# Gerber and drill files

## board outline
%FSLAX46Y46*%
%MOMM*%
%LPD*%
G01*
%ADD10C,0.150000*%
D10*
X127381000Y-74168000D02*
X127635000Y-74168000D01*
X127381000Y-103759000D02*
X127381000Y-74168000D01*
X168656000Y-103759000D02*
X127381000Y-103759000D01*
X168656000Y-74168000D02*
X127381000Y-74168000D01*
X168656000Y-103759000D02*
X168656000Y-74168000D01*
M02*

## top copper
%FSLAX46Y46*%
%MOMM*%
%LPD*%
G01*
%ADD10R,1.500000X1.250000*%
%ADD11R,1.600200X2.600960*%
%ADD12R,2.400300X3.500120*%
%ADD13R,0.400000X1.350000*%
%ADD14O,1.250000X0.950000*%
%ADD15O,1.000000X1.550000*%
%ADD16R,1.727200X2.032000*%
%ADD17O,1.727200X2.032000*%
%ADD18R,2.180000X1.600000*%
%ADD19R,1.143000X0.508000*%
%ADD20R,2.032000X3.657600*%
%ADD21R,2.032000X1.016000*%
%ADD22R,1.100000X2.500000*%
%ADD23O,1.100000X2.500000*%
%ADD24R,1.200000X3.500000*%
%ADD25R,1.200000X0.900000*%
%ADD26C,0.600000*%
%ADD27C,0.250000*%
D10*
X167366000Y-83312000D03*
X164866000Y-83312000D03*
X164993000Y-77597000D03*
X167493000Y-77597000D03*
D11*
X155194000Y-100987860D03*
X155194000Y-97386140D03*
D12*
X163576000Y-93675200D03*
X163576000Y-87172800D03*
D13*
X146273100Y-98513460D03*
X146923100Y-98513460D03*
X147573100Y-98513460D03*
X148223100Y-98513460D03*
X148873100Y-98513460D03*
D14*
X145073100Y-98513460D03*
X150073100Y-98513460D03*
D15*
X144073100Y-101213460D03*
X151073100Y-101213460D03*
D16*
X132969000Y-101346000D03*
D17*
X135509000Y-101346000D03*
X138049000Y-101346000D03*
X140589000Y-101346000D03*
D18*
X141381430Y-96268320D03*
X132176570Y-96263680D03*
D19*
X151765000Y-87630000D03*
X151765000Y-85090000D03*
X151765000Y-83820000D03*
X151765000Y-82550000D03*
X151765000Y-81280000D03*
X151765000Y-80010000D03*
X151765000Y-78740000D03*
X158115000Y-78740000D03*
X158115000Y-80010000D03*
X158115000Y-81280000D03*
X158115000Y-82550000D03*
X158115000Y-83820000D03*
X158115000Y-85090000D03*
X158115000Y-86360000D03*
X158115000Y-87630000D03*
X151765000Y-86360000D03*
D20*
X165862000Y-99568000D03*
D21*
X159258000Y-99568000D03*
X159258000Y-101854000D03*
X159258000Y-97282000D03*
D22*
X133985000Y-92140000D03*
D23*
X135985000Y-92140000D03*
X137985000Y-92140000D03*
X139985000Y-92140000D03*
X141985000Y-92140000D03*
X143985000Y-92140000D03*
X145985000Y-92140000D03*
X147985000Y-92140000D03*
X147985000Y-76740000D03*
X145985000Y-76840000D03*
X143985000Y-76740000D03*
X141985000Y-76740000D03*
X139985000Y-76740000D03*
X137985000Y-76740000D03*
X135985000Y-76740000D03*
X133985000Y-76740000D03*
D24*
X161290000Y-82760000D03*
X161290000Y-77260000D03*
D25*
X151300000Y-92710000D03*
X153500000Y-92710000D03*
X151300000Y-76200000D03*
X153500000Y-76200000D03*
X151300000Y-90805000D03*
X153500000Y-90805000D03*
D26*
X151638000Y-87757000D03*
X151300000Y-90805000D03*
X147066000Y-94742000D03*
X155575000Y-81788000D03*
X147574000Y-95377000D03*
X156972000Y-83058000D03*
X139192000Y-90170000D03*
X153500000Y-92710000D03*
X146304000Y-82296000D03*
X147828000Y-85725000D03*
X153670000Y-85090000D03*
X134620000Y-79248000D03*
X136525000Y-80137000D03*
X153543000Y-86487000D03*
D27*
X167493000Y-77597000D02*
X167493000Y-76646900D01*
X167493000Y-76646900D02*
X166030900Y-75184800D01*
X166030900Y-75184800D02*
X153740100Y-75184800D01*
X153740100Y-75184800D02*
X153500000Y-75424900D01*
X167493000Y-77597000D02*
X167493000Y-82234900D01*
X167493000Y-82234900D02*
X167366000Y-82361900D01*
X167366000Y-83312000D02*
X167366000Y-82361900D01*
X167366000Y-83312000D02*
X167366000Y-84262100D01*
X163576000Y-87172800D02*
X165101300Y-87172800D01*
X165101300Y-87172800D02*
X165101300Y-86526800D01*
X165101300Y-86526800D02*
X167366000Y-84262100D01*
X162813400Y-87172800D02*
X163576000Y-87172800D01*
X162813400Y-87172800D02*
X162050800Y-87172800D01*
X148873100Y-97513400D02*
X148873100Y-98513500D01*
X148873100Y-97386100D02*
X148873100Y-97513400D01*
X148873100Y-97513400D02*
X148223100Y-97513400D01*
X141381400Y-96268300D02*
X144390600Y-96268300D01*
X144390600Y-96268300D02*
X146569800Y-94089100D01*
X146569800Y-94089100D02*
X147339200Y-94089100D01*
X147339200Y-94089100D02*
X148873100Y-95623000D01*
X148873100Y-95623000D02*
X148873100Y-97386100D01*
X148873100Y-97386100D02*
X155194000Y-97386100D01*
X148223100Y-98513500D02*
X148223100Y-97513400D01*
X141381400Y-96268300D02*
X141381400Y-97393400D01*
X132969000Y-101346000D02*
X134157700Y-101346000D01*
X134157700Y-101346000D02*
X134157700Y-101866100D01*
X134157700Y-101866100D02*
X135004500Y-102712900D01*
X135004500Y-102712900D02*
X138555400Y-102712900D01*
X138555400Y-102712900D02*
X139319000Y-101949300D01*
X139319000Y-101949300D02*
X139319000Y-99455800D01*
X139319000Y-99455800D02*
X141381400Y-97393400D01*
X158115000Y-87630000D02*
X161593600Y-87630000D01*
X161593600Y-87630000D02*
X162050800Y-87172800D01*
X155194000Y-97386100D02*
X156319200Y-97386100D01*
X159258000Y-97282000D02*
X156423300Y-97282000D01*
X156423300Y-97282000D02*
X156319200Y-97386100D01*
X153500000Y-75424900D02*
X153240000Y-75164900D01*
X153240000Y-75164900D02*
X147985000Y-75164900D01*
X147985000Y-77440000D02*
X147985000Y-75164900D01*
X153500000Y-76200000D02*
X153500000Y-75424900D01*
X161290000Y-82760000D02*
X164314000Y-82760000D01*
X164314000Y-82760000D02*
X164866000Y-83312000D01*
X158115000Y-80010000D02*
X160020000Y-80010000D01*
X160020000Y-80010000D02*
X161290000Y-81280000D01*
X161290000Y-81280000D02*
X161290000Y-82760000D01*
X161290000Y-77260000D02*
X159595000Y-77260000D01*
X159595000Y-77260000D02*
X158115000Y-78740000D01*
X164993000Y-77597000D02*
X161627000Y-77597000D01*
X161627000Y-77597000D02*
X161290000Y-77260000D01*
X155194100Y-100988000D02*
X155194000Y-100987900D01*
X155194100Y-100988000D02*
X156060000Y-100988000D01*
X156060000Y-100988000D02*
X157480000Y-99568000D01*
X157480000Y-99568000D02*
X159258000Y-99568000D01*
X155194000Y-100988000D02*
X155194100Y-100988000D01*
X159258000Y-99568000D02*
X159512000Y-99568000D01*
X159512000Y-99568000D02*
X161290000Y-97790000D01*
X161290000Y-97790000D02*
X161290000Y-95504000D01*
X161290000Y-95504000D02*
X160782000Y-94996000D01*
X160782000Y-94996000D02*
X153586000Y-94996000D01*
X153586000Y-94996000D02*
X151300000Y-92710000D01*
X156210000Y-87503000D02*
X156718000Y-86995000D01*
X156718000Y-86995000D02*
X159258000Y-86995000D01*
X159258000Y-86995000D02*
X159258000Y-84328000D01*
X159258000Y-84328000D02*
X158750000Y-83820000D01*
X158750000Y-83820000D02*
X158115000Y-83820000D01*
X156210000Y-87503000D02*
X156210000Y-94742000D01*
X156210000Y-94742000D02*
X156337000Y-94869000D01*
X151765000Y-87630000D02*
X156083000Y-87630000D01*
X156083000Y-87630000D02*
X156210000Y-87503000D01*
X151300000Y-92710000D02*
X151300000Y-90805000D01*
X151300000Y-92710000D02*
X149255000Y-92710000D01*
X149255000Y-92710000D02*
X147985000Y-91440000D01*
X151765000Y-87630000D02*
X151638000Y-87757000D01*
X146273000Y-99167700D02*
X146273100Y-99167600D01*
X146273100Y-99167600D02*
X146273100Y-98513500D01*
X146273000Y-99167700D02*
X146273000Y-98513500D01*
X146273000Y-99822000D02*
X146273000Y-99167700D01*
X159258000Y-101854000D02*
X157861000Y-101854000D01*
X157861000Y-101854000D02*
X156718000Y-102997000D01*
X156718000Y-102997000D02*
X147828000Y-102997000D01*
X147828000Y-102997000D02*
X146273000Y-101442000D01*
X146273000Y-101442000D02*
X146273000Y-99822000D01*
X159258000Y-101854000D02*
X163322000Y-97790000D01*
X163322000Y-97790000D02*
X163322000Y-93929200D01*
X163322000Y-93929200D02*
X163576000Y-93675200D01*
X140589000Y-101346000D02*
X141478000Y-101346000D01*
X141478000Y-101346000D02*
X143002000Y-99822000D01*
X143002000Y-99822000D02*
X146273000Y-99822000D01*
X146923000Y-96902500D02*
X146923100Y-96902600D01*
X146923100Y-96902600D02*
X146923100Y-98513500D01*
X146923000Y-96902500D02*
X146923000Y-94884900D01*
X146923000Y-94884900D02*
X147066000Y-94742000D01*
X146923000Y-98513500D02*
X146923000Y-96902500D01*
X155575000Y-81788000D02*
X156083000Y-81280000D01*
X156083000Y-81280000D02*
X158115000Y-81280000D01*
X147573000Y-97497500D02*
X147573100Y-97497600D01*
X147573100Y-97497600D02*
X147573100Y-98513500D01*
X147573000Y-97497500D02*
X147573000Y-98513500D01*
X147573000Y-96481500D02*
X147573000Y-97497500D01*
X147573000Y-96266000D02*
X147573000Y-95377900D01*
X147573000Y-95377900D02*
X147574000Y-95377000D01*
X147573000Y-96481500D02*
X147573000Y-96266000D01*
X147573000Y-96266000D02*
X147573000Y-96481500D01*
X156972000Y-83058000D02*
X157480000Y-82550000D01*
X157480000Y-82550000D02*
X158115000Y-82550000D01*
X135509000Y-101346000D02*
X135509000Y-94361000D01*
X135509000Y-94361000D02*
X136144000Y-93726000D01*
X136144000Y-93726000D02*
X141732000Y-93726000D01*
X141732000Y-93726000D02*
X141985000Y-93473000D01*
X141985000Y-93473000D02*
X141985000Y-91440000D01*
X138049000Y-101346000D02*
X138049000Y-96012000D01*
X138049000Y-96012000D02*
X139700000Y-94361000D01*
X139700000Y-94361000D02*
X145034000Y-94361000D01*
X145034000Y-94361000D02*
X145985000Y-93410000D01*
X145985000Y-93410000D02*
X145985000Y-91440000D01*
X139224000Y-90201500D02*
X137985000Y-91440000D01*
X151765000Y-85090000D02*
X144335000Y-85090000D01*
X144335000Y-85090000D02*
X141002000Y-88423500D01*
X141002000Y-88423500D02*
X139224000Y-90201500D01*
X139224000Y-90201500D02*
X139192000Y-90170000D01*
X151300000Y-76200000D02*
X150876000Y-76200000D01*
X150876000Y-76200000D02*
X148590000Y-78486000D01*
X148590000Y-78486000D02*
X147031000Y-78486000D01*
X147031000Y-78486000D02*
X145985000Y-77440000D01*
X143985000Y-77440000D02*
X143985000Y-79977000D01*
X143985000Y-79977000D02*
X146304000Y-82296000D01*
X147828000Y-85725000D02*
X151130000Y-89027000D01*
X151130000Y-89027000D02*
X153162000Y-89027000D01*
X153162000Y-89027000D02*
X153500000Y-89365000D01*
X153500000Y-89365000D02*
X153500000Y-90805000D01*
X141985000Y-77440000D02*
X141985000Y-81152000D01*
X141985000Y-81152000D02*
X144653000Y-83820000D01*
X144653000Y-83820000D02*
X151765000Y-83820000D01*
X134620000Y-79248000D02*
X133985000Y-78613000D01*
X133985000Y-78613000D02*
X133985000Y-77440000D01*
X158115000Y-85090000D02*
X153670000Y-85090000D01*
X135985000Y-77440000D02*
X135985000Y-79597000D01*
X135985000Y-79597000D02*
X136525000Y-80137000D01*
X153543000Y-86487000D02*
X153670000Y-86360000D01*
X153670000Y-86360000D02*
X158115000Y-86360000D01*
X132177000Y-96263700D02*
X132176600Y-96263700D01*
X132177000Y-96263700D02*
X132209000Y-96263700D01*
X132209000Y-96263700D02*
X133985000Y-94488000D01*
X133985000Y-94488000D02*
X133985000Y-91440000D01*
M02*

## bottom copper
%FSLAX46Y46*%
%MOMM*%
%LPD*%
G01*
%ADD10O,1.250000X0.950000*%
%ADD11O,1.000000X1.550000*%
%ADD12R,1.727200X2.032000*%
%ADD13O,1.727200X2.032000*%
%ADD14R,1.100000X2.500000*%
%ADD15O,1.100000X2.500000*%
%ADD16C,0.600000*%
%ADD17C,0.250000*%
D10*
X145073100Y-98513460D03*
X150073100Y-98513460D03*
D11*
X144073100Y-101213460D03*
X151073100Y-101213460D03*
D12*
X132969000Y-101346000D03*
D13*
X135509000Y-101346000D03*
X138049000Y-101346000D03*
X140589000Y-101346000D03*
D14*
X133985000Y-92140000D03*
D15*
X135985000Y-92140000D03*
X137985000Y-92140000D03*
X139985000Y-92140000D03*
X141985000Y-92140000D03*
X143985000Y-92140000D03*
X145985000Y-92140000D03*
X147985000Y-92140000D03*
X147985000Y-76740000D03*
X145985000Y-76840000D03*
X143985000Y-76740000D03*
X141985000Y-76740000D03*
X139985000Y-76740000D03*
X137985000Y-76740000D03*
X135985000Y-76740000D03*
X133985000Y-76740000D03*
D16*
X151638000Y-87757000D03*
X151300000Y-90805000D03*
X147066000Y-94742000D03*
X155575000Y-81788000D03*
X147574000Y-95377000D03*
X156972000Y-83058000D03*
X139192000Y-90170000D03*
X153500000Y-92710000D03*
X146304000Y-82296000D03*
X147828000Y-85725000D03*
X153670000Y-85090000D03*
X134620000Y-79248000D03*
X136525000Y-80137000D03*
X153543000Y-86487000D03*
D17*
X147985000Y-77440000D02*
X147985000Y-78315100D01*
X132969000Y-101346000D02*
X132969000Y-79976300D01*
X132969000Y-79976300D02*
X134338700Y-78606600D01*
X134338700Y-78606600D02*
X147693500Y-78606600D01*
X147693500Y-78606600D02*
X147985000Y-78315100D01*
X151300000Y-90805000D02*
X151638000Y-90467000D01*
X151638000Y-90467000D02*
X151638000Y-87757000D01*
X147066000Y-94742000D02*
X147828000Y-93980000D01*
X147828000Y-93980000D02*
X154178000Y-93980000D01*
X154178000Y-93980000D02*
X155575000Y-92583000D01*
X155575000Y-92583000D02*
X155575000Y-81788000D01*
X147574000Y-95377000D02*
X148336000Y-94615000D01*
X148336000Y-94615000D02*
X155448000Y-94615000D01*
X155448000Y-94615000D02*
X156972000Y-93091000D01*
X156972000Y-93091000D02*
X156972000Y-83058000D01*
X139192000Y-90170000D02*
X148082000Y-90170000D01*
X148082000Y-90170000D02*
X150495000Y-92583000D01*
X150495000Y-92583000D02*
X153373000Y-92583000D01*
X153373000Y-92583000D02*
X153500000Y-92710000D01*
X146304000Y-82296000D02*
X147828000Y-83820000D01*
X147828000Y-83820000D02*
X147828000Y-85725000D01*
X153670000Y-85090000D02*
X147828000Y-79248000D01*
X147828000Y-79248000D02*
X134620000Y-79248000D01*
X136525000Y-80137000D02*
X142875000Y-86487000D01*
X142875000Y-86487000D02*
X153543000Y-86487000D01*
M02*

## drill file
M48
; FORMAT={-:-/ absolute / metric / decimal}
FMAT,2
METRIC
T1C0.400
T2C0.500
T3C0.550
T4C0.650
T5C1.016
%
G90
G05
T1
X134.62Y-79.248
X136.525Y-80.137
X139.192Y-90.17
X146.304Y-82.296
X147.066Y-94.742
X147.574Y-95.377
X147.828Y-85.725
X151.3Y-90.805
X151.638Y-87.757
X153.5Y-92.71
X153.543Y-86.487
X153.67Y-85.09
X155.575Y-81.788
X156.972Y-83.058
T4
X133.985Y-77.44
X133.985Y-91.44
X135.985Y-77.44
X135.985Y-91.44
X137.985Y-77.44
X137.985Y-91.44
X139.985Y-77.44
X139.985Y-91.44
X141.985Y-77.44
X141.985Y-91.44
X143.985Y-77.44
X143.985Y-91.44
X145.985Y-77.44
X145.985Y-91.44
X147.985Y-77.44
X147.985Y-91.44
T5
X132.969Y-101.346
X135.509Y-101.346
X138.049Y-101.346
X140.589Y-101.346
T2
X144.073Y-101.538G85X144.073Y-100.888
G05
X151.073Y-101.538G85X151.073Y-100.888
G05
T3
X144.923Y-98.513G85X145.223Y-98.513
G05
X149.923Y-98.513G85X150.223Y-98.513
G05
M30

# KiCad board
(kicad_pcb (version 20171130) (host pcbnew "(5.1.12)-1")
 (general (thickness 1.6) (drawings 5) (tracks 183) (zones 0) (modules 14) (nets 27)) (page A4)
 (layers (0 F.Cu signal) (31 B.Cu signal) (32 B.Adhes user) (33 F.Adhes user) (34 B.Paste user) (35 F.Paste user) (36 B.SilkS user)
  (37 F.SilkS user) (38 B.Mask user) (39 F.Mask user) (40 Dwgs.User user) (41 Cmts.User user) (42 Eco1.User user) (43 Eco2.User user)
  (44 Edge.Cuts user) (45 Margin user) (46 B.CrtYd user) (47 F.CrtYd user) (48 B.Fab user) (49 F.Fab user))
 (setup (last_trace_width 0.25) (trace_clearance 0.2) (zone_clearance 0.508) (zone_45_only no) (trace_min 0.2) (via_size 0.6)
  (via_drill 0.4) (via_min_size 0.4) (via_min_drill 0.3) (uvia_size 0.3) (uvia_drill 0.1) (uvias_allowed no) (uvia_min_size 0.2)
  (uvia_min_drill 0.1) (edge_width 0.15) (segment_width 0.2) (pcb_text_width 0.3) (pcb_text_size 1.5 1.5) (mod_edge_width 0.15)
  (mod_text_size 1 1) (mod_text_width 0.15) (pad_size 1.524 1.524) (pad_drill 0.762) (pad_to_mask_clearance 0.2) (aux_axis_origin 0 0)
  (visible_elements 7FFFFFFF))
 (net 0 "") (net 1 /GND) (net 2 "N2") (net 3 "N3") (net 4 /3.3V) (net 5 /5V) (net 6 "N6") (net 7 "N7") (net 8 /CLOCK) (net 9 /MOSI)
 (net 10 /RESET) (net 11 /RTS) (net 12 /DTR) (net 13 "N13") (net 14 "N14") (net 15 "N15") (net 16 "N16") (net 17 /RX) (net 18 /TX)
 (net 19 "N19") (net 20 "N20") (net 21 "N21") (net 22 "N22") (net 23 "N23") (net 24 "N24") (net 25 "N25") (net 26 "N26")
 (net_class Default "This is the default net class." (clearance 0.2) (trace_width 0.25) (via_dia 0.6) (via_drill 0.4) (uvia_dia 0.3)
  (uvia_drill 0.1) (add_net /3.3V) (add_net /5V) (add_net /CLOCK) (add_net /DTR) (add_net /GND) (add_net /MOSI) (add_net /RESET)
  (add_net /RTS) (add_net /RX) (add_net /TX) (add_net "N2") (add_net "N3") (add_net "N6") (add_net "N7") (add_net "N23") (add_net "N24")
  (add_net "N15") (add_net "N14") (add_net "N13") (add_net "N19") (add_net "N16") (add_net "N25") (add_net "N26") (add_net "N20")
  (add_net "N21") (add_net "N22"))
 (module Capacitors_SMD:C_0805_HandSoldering (layer F.Cu) (at 166.116 83.312 180)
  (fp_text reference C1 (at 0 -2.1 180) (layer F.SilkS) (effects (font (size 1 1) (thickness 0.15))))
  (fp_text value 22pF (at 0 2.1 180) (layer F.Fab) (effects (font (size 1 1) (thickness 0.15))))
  (pad 1 smd rect (at -1.25 0 180) (size 1.5 1.25) (layers F.Cu F.Paste F.Mask) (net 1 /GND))
  (pad 2 smd rect (at 1.25 0 180) (size 1.5 1.25) (layers F.Cu F.Paste F.Mask) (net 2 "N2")))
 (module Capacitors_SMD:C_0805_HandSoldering (layer F.Cu) (at 166.243 77.597)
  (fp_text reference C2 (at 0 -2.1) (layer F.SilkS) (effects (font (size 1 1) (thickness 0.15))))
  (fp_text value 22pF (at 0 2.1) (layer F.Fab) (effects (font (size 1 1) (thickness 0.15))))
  (pad 1 smd rect (at -1.25 0) (size 1.5 1.25) (layers F.Cu F.Paste F.Mask) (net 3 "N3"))
  (pad 2 smd rect (at 1.25 0) (size 1.5 1.25) (layers F.Cu F.Paste F.Mask) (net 1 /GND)))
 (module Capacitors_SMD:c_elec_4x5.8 (layer F.Cu) (at 155.194 99.187 270)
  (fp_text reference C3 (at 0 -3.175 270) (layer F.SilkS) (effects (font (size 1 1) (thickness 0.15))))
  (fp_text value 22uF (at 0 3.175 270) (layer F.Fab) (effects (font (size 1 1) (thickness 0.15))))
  (pad 1 smd rect (at 1.80086 0 270) (size 2.60096 1.6002) (layers F.Cu F.Paste F.Mask) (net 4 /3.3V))
  (pad 2 smd rect (at -1.80086 0 270) (size 2.60096 1.6002) (layers F.Cu F.Paste F.Mask) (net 1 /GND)))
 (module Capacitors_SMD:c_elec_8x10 (layer F.Cu) (at 163.576 90.424 270)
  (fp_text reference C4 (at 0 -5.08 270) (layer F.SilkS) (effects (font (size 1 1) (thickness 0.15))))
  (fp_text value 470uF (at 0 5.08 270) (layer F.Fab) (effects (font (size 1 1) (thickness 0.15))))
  (pad 1 smd rect (at 3.2512 0 270) (size 3.50012 2.4003) (layers F.Cu F.Paste F.Mask) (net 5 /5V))
  (pad 2 smd rect (at -3.2512 0 270) (size 3.50012 2.4003) (layers F.Cu F.Paste F.Mask) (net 1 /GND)))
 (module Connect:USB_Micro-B (layer F.Cu) (at 147.574 100.076)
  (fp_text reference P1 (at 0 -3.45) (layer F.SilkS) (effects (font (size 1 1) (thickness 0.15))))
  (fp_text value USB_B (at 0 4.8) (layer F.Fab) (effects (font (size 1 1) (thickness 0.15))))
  (pad 1 smd rect (at -1.3009 -1.56254 90) (size 1.35 0.4) (layers F.Cu F.Paste F.Mask) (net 5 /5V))
  (pad 2 smd rect (at -0.6509 -1.56254 90) (size 1.35 0.4) (layers F.Cu F.Paste F.Mask) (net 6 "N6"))
  (pad 3 smd rect (at -0.0009 -1.56254 90) (size 1.35 0.4) (layers F.Cu F.Paste F.Mask) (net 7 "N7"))
  (pad 4 smd rect (at 0.6491 -1.56254 90) (size 1.35 0.4) (layers F.Cu F.Paste F.Mask) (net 1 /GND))
  (pad 5 smd rect (at 1.2991 -1.56254 90) (size 1.35 0.4) (layers F.Cu F.Paste F.Mask) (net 1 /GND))
  (pad 6 thru_hole oval (at -2.5009 -1.56254 90) (size 0.95 1.25) (drill oval 0.55 0.85) (layers *.Cu *.Mask F.SilkS))
  (pad 6 thru_hole oval (at 2.4991 -1.56254 90) (size 0.95 1.25) (drill oval 0.55 0.85) (layers *.Cu *.Mask F.SilkS))
  (pad 6 thru_hole oval (at -3.5009 1.13746 90) (size 1.55 1) (drill oval 1.15 0.5) (layers *.Cu *.Mask F.SilkS))
  (pad 6 thru_hole oval (at 3.4991 1.13746 90) (size 1.55 1) (drill oval 1.15 0.5) (layers *.Cu *.Mask F.SilkS)))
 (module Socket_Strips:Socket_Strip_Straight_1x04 (layer F.Cu) (at 132.969 101.346)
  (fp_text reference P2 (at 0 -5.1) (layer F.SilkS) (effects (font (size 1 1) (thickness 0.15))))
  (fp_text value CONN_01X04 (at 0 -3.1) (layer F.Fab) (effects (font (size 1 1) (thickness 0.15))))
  (pad 1 thru_hole rect (at 0 0) (size 1.7272 2.032) (drill 1.016) (layers *.Cu *.Mask F.SilkS) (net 1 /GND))
  (pad 2 thru_hole oval (at 2.54 0) (size 1.7272 2.032) (drill 1.016) (layers *.Cu *.Mask F.SilkS) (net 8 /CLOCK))
  (pad 3 thru_hole oval (at 5.08 0) (size 1.7272 2.032) (drill 1.016) (layers *.Cu *.Mask F.SilkS) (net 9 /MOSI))
  (pad 4 thru_hole oval (at 7.62 0) (size 1.7272 2.032) (drill 1.016) (layers *.Cu *.Mask F.SilkS) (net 5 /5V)))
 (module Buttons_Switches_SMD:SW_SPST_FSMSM (layer F.Cu) (at 136.779 96.266 180)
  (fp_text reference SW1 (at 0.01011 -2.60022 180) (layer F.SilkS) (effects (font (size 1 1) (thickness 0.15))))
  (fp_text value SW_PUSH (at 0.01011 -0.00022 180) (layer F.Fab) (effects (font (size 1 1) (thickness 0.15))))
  (pad 1 smd rect (at -4.60243 -0.00232 180) (size 2.18 1.6) (layers F.Cu F.Paste F.Mask) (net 1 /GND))
  (pad 2 smd rect (at 4.60243 0.00232 180) (size 2.18 1.6) (layers F.Cu F.Paste F.Mask) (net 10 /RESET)))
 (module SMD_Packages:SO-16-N (layer F.Cu) (at 154.94 83.185 90)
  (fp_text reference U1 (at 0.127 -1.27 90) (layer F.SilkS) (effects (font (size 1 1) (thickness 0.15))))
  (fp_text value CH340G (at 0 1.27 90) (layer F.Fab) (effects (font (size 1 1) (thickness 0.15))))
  (pad 16 smd rect (at -4.445 -3.175 90) (size 0.508 1.143) (layers F.Cu F.Paste F.Mask) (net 4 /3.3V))
  (pad 14 smd rect (at -1.905 -3.175 90) (size 0.508 1.143) (layers F.Cu F.Paste F.Mask) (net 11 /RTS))
  (pad 13 smd rect (at -0.635 -3.175 90) (size 0.508 1.143) (layers F.Cu F.Paste F.Mask) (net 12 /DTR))
  (pad 12 smd rect (at 0.635 -3.175 90) (size 0.508 1.143) (layers F.Cu F.Paste F.Mask) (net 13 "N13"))
  (pad 11 smd rect (at 1.905 -3.175 90) (size 0.508 1.143) (layers F.Cu F.Paste F.Mask) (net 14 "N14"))
  (pad 10 smd rect (at 3.175 -3.175 90) (size 0.508 1.143) (layers F.Cu F.Paste F.Mask) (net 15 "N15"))
  (pad 9 smd rect (at 4.445 -3.175 90) (size 0.508 1.143) (layers F.Cu F.Paste F.Mask) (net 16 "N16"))
  (pad 8 smd rect (at 4.445 3.175 90) (size 0.508 1.143) (layers F.Cu F.Paste F.Mask) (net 3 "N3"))
  (pad 7 smd rect (at 3.175 3.175 90) (size 0.508 1.143) (layers F.Cu F.Paste F.Mask) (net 2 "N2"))
  (pad 6 smd rect (at 1.905 3.175 90) (size 0.508 1.143) (layers F.Cu F.Paste F.Mask) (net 6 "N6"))
  (pad 5 smd rect (at 0.635 3.175 90) (size 0.508 1.143) (layers F.Cu F.Paste F.Mask) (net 7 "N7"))
  (pad 4 smd rect (at -0.635 3.175 90) (size 0.508 1.143) (layers F.Cu F.Paste F.Mask) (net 4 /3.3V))
  (pad 3 smd rect (at -1.905 3.175 90) (size 0.508 1.143) (layers F.Cu F.Paste F.Mask) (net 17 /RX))
  (pad 2 smd rect (at -3.175 3.175 90) (size 0.508 1.143) (layers F.Cu F.Paste F.Mask) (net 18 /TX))
  (pad 1 smd rect (at -4.445 3.175 90) (size 0.508 1.143) (layers F.Cu F.Paste F.Mask) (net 1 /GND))
  (pad 15 smd rect (at -3.175 -3.175 90) (size 0.508 1.143) (layers F.Cu F.Paste F.Mask) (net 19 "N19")))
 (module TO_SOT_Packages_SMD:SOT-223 (layer F.Cu) (at 162.56 99.568 270)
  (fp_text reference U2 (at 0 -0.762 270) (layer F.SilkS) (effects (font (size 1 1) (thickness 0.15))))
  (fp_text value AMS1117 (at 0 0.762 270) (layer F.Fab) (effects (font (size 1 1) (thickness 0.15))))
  (pad 4 smd rect (at 0 -3.302 270) (size 3.6576 2.032) (layers F.Cu F.Paste F.Mask))
  (pad 2 smd rect (at 0 3.302 270) (size 1.016 2.032) (layers F.Cu F.Paste F.Mask) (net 4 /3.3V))
  (pad 3 smd rect (at 2.286 3.302 270) (size 1.016 2.032) (layers F.Cu F.Paste F.Mask) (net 5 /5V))
  (pad 1 smd rect (at -2.286 3.302 270) (size 1.016 2.032) (layers F.Cu F.Paste F.Mask) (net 1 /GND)))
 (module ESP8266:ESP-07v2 (layer F.Cu) (at 133.985 91.44 90)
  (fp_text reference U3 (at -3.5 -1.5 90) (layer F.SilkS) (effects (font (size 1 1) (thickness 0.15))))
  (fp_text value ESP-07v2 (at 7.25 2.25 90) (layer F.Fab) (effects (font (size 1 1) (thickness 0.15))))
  (pad 1 thru_hole rect (at 0 0 90) (size 2.5 1.1) (drill 0.65 (offset -0.7 0)) (layers *.Cu *.Mask F.SilkS) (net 10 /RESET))
  (pad 2 thru_hole oval (at 0 2 90) (size 2.5 1.1) (drill 0.65 (offset -0.7 0)) (layers *.Cu *.Mask F.SilkS) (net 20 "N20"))
  (pad 3 thru_hole oval (at 0 4 90) (size 2.5 1.1) (drill 0.65 (offset -0.7 0)) (layers *.Cu *.Mask F.SilkS) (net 11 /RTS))
  (pad 4 thru_hole oval (at 0 6 90) (size 2.5 1.1) (drill 0.65 (offset -0.7 0)) (layers *.Cu *.Mask F.SilkS) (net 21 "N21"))
  (pad 5 thru_hole oval (at 0 8 90) (size 2.5 1.1) (drill 0.65 (offset -0.7 0)) (layers *.Cu *.Mask F.SilkS) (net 8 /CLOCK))
  (pad 6 thru_hole oval (at 0 10 90) (size 2.5 1.1) (drill 0.65 (offset -0.7 0)) (layers *.Cu *.Mask F.SilkS) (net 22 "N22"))
  (pad 7 thru_hole oval (at 0 12 90) (size 2.5 1.1) (drill 0.65 (offset -0.7 0)) (layers *.Cu *.Mask F.SilkS) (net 9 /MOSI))
  (pad 8 thru_hole oval (at 0 14 90) (size 2.5 1.1) (drill 0.65 (offset -0.7 0)) (layers *.Cu *.Mask F.SilkS) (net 4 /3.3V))
  (pad 9 thru_hole oval (at 14 14 90) (size 2.5 1.1) (drill 0.65 (offset 0.7 0)) (layers *.Cu *.Mask F.SilkS) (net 1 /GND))
  (pad 10 thru_hole oval (at 14 12 90) (size 2.5 1.1) (drill 0.65 (offset 0.6 0)) (layers *.Cu *.Mask F.SilkS) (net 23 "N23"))
  (pad 11 thru_hole oval (at 14 10 90) (size 2.5 1.1) (drill 0.65 (offset 0.7 0)) (layers *.Cu *.Mask F.SilkS) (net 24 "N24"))
  (pad 12 thru_hole oval (at 14 8 90) (size 2.5 1.1) (drill 0.65 (offset 0.7 0)) (layers *.Cu *.Mask F.SilkS) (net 12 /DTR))
  (pad 13 thru_hole oval (at 14 6 90) (size 2.5 1.1) (drill 0.65 (offset 0.7 0)) (layers *.Cu *.Mask F.SilkS) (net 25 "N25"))
  (pad 14 thru_hole oval (at 14 4 90) (size 2.5 1.1) (drill 0.65 (offset 0.7 0)) (layers *.Cu *.Mask F.SilkS) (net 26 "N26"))
  (pad 15 thru_hole oval (at 14 2 90) (size 2.5 1.1) (drill 0.65 (offset 0.7 0)) (layers *.Cu *.Mask F.SilkS) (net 18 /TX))
  (pad 16 thru_hole oval (at 14 0 90) (size 2.5 1.1) (drill 0.65 (offset 0.7 0)) (layers *.Cu *.Mask F.SilkS) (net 17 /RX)))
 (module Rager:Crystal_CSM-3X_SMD (layer F.Cu) (at 161.29 80.01 90)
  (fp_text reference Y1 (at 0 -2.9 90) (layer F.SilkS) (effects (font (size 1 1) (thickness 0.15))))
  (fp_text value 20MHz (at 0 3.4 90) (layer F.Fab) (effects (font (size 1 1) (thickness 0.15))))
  (pad 1 smd rect (at -2.75 0 90) (size 3.5 1.2) (layers F.Cu F.Paste F.Mask) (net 2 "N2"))
  (pad 2 smd rect (at 2.75 0 90) (size 3.5 1.2) (layers F.Cu F.Paste F.Mask) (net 3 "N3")))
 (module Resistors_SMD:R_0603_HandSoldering (layer F.Cu) (at 152.4 92.71)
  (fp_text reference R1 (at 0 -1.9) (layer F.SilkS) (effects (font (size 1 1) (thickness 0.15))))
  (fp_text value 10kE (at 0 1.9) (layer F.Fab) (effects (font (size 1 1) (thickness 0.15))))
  (pad 1 smd rect (at -1.1 0) (size 1.2 0.9) (layers F.Cu F.Paste F.Mask) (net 4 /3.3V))
  (pad 2 smd rect (at 1.1 0) (size 1.2 0.9) (layers F.Cu F.Paste F.Mask) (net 11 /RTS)))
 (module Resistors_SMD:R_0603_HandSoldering (layer F.Cu) (at 152.4 76.2)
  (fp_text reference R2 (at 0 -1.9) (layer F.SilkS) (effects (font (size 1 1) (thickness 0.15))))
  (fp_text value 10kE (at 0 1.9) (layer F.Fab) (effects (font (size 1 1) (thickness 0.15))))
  (pad 1 smd rect (at -1.1 0) (size 1.2 0.9) (layers F.Cu F.Paste F.Mask) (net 23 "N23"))
  (pad 2 smd rect (at 1.1 0) (size 1.2 0.9) (layers F.Cu F.Paste F.Mask) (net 1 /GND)))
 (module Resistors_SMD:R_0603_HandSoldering (layer F.Cu) (at 152.4 90.805)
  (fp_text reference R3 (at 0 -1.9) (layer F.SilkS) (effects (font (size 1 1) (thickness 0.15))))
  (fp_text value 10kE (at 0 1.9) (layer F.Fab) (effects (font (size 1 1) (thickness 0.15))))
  (pad 1 smd rect (at -1.1 0) (size 1.2 0.9) (layers F.Cu F.Paste F.Mask) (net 4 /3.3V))
  (pad 2 smd rect (at 1.1 0) (size 1.2 0.9) (layers F.Cu F.Paste F.Mask) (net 24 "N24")))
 (gr_line (start 127.381 74.168) (end 127.635 74.168) (angle 90) (layer Edge.Cuts) (width 0.15))
 (gr_line (start 127.381 103.759) (end 127.381 74.168) (angle 90) (layer Edge.Cuts) (width 0.15))
 (gr_line (start 168.656 103.759) (end 127.381 103.759) (angle 90) (layer Edge.Cuts) (width 0.15))
 (gr_line (start 168.656 74.168) (end 127.381 74.168) (angle 90) (layer Edge.Cuts) (width 0.15))
 (gr_line (start 168.656 103.759) (end 168.656 74.168) (angle 90) (layer Edge.Cuts) (width 0.15))
 (segment (start 167.493 77.597) (end 167.493 76.6469) (width 0.25) (layer F.Cu) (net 1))
 (segment (start 167.493 76.6469) (end 166.0309 75.1848) (width 0.25) (layer F.Cu) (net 1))
 (segment (start 166.0309 75.1848) (end 153.7401 75.1848) (width 0.25) (layer F.Cu) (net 1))
 (segment (start 153.7401 75.1848) (end 153.5 75.4249) (width 0.25) (layer F.Cu) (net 1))
 (segment (start 167.493 77.597) (end 167.493 82.2349) (width 0.25) (layer F.Cu) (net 1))
 (segment (start 167.493 82.2349) (end 167.366 82.3619) (width 0.25) (layer F.Cu) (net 1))
 (segment (start 167.366 83.312) (end 167.366 82.3619) (width 0.25) (layer F.Cu) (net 1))
 (segment (start 147.985 77.44) (end 147.985 78.3151) (width 0.25) (layer B.Cu) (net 1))
 (segment (start 132.969 101.346) (end 132.969 79.9763) (width 0.25) (layer B.Cu) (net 1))
 (segment (start 132.969 79.9763) (end 134.3387 78.6066) (width 0.25) (layer B.Cu) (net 1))
 (segment (start 134.3387 78.6066) (end 147.6935 78.6066) (width 0.25) (layer B.Cu) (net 1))
 (segment (start 147.6935 78.6066) (end 147.985 78.3151) (width 0.25) (layer B.Cu) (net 1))
 (segment (start 167.366 83.312) (end 167.366 84.2621) (width 0.25) (layer F.Cu) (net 1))
 (segment (start 163.576 87.1728) (end 165.1013 87.1728) (width 0.25) (layer F.Cu) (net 1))
 (segment (start 165.1013 87.1728) (end 165.1013 86.5268) (width 0.25) (layer F.Cu) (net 1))
 (segment (start 165.1013 86.5268) (end 167.366 84.2621) (width 0.25) (layer F.Cu) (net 1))
 (segment (start 162.8134 87.1728) (end 163.576 87.1728) (width 0.25) (layer F.Cu) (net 1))
 (segment (start 162.8134 87.1728) (end 162.0508 87.1728) (width 0.25) (layer F.Cu) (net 1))
 (segment (start 148.8731 97.5134) (end 148.8731 98.5135) (width 0.25) (layer F.Cu) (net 1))
 (segment (start 148.8731 97.3861) (end 148.8731 97.5134) (width 0.25) (layer F.Cu) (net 1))
 (segment (start 148.8731 97.5134) (end 148.2231 97.5134) (width 0.25) (layer F.Cu) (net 1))
 (segment (start 141.3814 96.2683) (end 144.3906 96.2683) (width 0.25) (layer F.Cu) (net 1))
 (segment (start 144.3906 96.2683) (end 146.5698 94.0891) (width 0.25) (layer F.Cu) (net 1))
 (segment (start 146.5698 94.0891) (end 147.3392 94.0891) (width 0.25) (layer F.Cu) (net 1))
 (segment (start 147.3392 94.0891) (end 148.8731 95.623) (width 0.25) (layer F.Cu) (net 1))
 (segment (start 148.8731 95.623) (end 148.8731 97.3861) (width 0.25) (layer F.Cu) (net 1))
 (segment (start 148.8731 97.3861) (end 155.194 97.3861) (width 0.25) (layer F.Cu) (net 1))
 (segment (start 148.2231 98.5135) (end 148.2231 97.5134) (width 0.25) (layer F.Cu) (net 1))
 (segment (start 141.3814 96.2683) (end 141.3814 97.3934) (width 0.25) (layer F.Cu) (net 1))
 (segment (start 132.969 101.346) (end 134.1577 101.346) (width 0.25) (layer F.Cu) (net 1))
 (segment (start 134.1577 101.346) (end 134.1577 101.8661) (width 0.25) (layer F.Cu) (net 1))
 (segment (start 134.1577 101.8661) (end 135.0045 102.7129) (width 0.25) (layer F.Cu) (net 1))
 (segment (start 135.0045 102.7129) (end 138.5554 102.7129) (width 0.25) (layer F.Cu) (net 1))
 (segment (start 138.5554 102.7129) (end 139.319 101.9493) (width 0.25) (layer F.Cu) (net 1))
 (segment (start 139.319 101.9493) (end 139.319 99.4558) (width 0.25) (layer F.Cu) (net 1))
 (segment (start 139.319 99.4558) (end 141.3814 97.3934) (width 0.25) (layer F.Cu) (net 1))
 (segment (start 158.115 87.63) (end 161.5936 87.63) (width 0.25) (layer F.Cu) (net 1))
 (segment (start 161.5936 87.63) (end 162.0508 87.1728) (width 0.25) (layer F.Cu) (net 1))
 (segment (start 155.194 97.3861) (end 156.3192 97.3861) (width 0.25) (layer F.Cu) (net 1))
 (segment (start 159.258 97.282) (end 156.4233 97.282) (width 0.25) (layer F.Cu) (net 1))
 (segment (start 156.4233 97.282) (end 156.3192 97.3861) (width 0.25) (layer F.Cu) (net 1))
 (segment (start 153.5 75.4249) (end 153.24 75.1649) (width 0.25) (layer F.Cu) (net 1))
 (segment (start 153.24 75.1649) (end 147.985 75.1649) (width 0.25) (layer F.Cu) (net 1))
 (segment (start 147.985 77.44) (end 147.985 75.1649) (width 0.25) (layer F.Cu) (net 1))
 (segment (start 153.5 76.2) (end 153.5 75.4249) (width 0.25) (layer F.Cu) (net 1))
 (segment (start 161.29 82.76) (end 164.314 82.76) (width 0.25) (layer F.Cu) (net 2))
 (segment (start 164.314 82.76) (end 164.866 83.312) (width 0.25) (layer F.Cu) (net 2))
 (segment (start 158.115 80.01) (end 160.02 80.01) (width 0.25) (layer F.Cu) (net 2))
 (segment (start 160.02 80.01) (end 161.29 81.28) (width 0.25) (layer F.Cu) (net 2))
 (segment (start 161.29 81.28) (end 161.29 82.76) (width 0.25) (layer F.Cu) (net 2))
 (segment (start 161.29 77.26) (end 159.595 77.26) (width 0.25) (layer F.Cu) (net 3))
 (segment (start 159.595 77.26) (end 158.115 78.74) (width 0.25) (layer F.Cu) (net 3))
 (segment (start 164.993 77.597) (end 161.627 77.597) (width 0.25) (layer F.Cu) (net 3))
 (segment (start 161.627 77.597) (end 161.29 77.26) (width 0.25) (layer F.Cu) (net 3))
 (segment (start 155.1941 100.988) (end 155.194 100.9879) (width 0.25) (layer F.Cu) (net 4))
 (segment (start 155.1941 100.988) (end 156.06 100.988) (width 0.25) (layer F.Cu) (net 4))
 (segment (start 156.06 100.988) (end 157.48 99.568) (width 0.25) (layer F.Cu) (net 4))
 (segment (start 157.48 99.568) (end 159.258 99.568) (width 0.25) (layer F.Cu) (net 4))
 (segment (start 155.194 100.988) (end 155.1941 100.988) (width 0.25) (layer F.Cu) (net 4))
 (segment (start 159.258 99.568) (end 159.512 99.568) (width 0.25) (layer F.Cu) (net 4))
 (segment (start 159.512 99.568) (end 161.29 97.79) (width 0.25) (layer F.Cu) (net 4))
 (segment (start 161.29 97.79) (end 161.29 95.504) (width 0.25) (layer F.Cu) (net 4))
 (segment (start 161.29 95.504) (end 160.782 94.996) (width 0.25) (layer F.Cu) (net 4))
 (segment (start 160.782 94.996) (end 153.586 94.996) (width 0.25) (layer F.Cu) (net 4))
 (segment (start 153.586 94.996) (end 151.3 92.71) (width 0.25) (layer F.Cu) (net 4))
 (segment (start 156.21 87.503) (end 156.718 86.995) (width 0.25) (layer F.Cu) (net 4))
 (segment (start 156.718 86.995) (end 159.258 86.995) (width 0.25) (layer F.Cu) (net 4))
 (segment (start 159.258 86.995) (end 159.258 84.328) (width 0.25) (layer F.Cu) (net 4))
 (segment (start 159.258 84.328) (end 158.75 83.82) (width 0.25) (layer F.Cu) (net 4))
 (segment (start 158.75 83.82) (end 158.115 83.82) (width 0.25) (layer F.Cu) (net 4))
 (segment (start 156.21 87.503) (end 156.21 94.742) (width 0.25) (layer F.Cu) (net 4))
 (segment (start 156.21 94.742) (end 156.337 94.869) (width 0.25) (layer F.Cu) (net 4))
 (segment (start 151.765 87.63) (end 156.083 87.63) (width 0.25) (layer F.Cu) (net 4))
 (segment (start 156.083 87.63) (end 156.21 87.503) (width 0.25) (layer F.Cu) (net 4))
 (segment (start 151.3 92.71) (end 151.3 90.805) (width 0.25) (layer F.Cu) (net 4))
 (segment (start 151.3 92.71) (end 149.255 92.71) (width 0.25) (layer F.Cu) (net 4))
 (segment (start 149.255 92.71) (end 147.985 91.44) (width 0.25) (layer F.Cu) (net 4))
 (segment (start 151.765 87.63) (end 151.638 87.757) (width 0.25) (layer F.Cu) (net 4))
 (segment (start 151.3 90.805) (end 151.638 90.467) (width 0.25) (layer B.Cu) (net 4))
 (segment (start 151.638 90.467) (end 151.638 87.757) (width 0.25) (layer B.Cu) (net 4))
 (via (at 151.638 87.757) (size 0.6) (layers F.Cu B.Cu) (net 4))
 (via (at 151.3 90.805) (size 0.6) (layers F.Cu B.Cu) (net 4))
 (segment (start 146.273 99.1677) (end 146.2731 99.1676) (width 0.25) (layer F.Cu) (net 5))
 (segment (start 146.2731 99.1676) (end 146.2731 98.5135) (width 0.25) (layer F.Cu) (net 5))
 (segment (start 146.273 99.1677) (end 146.273 98.5135) (width 0.25) (layer F.Cu) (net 5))
 (segment (start 146.273 99.822) (end 146.273 99.1677) (width 0.25) (layer F.Cu) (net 5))
 (segment (start 159.258 101.854) (end 157.861 101.854) (width 0.25) (layer F.Cu) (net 5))
 (segment (start 157.861 101.854) (end 156.718 102.997) (width 0.25) (layer F.Cu) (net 5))
 (segment (start 156.718 102.997) (end 147.828 102.997) (width 0.25) (layer F.Cu) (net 5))
 (segment (start 147.828 102.997) (end 146.273 101.442) (width 0.25) (layer F.Cu) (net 5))
 (segment (start 146.273 101.442) (end 146.273 99.822) (width 0.25) (layer F.Cu) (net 5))
 (segment (start 159.258 101.854) (end 163.322 97.79) (width 0.25) (layer F.Cu) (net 5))
 (segment (start 163.322 97.79) (end 163.322 93.9292) (width 0.25) (layer F.Cu) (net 5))
 (segment (start 163.322 93.9292) (end 163.576 93.6752) (width 0.25) (layer F.Cu) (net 5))
 (segment (start 140.589 101.346) (end 141.478 101.346) (width 0.25) (layer F.Cu) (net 5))
 (segment (start 141.478 101.346) (end 143.002 99.822) (width 0.25) (layer F.Cu) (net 5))
 (segment (start 143.002 99.822) (end 146.273 99.822) (width 0.25) (layer F.Cu) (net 5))
 (segment (start 146.923 96.9025) (end 146.9231 96.9026) (width 0.25) (layer F.Cu) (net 6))
 (segment (start 146.9231 96.9026) (end 146.9231 98.5135) (width 0.25) (layer F.Cu) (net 6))
 (segment (start 146.923 96.9025) (end 146.923 94.8849) (width 0.25) (layer F.Cu) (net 6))
 (segment (start 146.923 94.8849) (end 147.066 94.742) (width 0.25) (layer F.Cu) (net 6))
 (segment (start 146.923 98.5135) (end 146.923 96.9025) (width 0.25) (layer F.Cu) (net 6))
 (segment (start 147.066 94.742) (end 147.828 93.98) (width 0.25) (layer B.Cu) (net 6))
 (segment (start 147.828 93.98) (end 154.178 93.98) (width 0.25) (layer B.Cu) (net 6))
 (segment (start 154.178 93.98) (end 155.575 92.583) (width 0.25) (layer B.Cu) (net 6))
 (segment (start 155.575 92.583) (end 155.575 81.788) (width 0.25) (layer B.Cu) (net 6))
 (segment (start 155.575 81.788) (end 156.083 81.28) (width 0.25) (layer F.Cu) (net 6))
 (segment (start 156.083 81.28) (end 158.115 81.28) (width 0.25) (layer F.Cu) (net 6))
 (via (at 147.066 94.742) (size 0.6) (layers F.Cu B.Cu) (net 6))
 (via (at 155.575 81.788) (size 0.6) (layers F.Cu B.Cu) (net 6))
 (segment (start 147.573 97.4975) (end 147.5731 97.4976) (width 0.25) (layer F.Cu) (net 7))
 (segment (start 147.5731 97.4976) (end 147.5731 98.5135) (width 0.25) (layer F.Cu) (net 7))
 (segment (start 147.573 97.4975) (end 147.573 98.5135) (width 0.25) (layer F.Cu) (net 7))
 (segment (start 147.573 96.4815) (end 147.573 97.4975) (width 0.25) (layer F.Cu) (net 7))
 (segment (start 147.573 96.266) (end 147.573 95.3779) (width 0.25) (layer F.Cu) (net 7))
 (segment (start 147.573 95.3779) (end 147.574 95.377) (width 0.25) (layer F.Cu) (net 7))
 (segment (start 147.573 96.4815) (end 147.573 96.266) (width 0.25) (layer F.Cu) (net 7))
 (segment (start 147.573 96.266) (end 147.573 96.4815) (width 0.25) (layer F.Cu) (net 7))
 (segment (start 147.574 95.377) (end 148.336 94.615) (width 0.25) (layer B.Cu) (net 7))
 (segment (start 148.336 94.615) (end 155.448 94.615) (width 0.25) (layer B.Cu) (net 7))
 (segment (start 155.448 94.615) (end 156.972 93.091) (width 0.25) (layer B.Cu) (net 7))
 (segment (start 156.972 93.091) (end 156.972 83.058) (width 0.25) (layer B.Cu) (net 7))
 (segment (start 156.972 83.058) (end 157.48 82.55) (width 0.25) (layer F.Cu) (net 7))
 (segment (start 157.48 82.55) (end 158.115 82.55) (width 0.25) (layer F.Cu) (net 7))
 (via (at 147.574 95.377) (size 0.6) (layers F.Cu B.Cu) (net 7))
 (via (at 156.972 83.058) (size 0.6) (layers F.Cu B.Cu) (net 7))
 (segment (start 135.509 101.346) (end 135.509 94.361) (width 0.25) (layer F.Cu) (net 8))
 (segment (start 135.509 94.361) (end 136.144 93.726) (width 0.25) (layer F.Cu) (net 8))
 (segment (start 136.144 93.726) (end 141.732 93.726) (width 0.25) (layer F.Cu) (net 8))
 (segment (start 141.732 93.726) (end 141.985 93.473) (width 0.25) (layer F.Cu) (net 8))
 (segment (start 141.985 93.473) (end 141.985 91.44) (width 0.25) (layer F.Cu) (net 8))
 (segment (start 138.049 101.346) (end 138.049 96.012) (width 0.25) (layer F.Cu) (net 9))
 (segment (start 138.049 96.012) (end 139.7 94.361) (width 0.25) (layer F.Cu) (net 9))
 (segment (start 139.7 94.361) (end 145.034 94.361) (width 0.25) (layer F.Cu) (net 9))
 (segment (start 145.034 94.361) (end 145.985 93.41) (width 0.25) (layer F.Cu) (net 9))
 (segment (start 145.985 93.41) (end 145.985 91.44) (width 0.25) (layer F.Cu) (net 9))
 (segment (start 139.224 90.2015) (end 137.985 91.44) (width 0.25) (layer F.Cu) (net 11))
 (segment (start 151.765 85.09) (end 144.335 85.09) (width 0.25) (layer F.Cu) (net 11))
 (segment (start 144.335 85.09) (end 141.002 88.4235) (width 0.25) (layer F.Cu) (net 11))
 (segment (start 141.002 88.4235) (end 139.224 90.2015) (width 0.25) (layer F.Cu) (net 11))
 (segment (start 139.192 90.17) (end 148.082 90.17) (width 0.25) (layer B.Cu) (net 11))
 (segment (start 148.082 90.17) (end 150.495 92.583) (width 0.25) (layer B.Cu) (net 11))
 (segment (start 150.495 92.583) (end 153.373 92.583) (width 0.25) (layer B.Cu) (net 11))
 (segment (start 153.373 92.583) (end 153.5 92.71) (width 0.25) (layer B.Cu) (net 11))
 (segment (start 139.224 90.2015) (end 139.192 90.17) (width 0.25) (layer F.Cu) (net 11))
 (via (at 139.192 90.17) (size 0.6) (layers F.Cu B.Cu) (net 11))
 (via (at 153.5 92.71) (size 0.6) (layers F.Cu B.Cu) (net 11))
 (segment (start 151.3 76.2) (end 150.876 76.2) (width 0.25) (layer F.Cu) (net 23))
 (segment (start 150.876 76.2) (end 148.59 78.486) (width 0.25) (layer F.Cu) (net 23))
 (segment (start 148.59 78.486) (end 147.031 78.486) (width 0.25) (layer F.Cu) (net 23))
 (segment (start 147.031 78.486) (end 145.985 77.44) (width 0.25) (layer F.Cu) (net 23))
 (segment (start 143.985 77.44) (end 143.985 79.977) (width 0.25) (layer F.Cu) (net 24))
 (segment (start 143.985 79.977) (end 146.304 82.296) (width 0.25) (layer F.Cu) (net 24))
 (segment (start 146.304 82.296) (end 147.828 83.82) (width 0.25) (layer B.Cu) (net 24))
 (segment (start 147.828 83.82) (end 147.828 85.725) (width 0.25) (layer B.Cu) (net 24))
 (segment (start 147.828 85.725) (end 151.13 89.027) (width 0.25) (layer F.Cu) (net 24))
 (segment (start 151.13 89.027) (end 153.162 89.027) (width 0.25) (layer F.Cu) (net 24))
 (segment (start 153.162 89.027) (end 153.5 89.365) (width 0.25) (layer F.Cu) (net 24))
 (segment (start 153.5 89.365) (end 153.5 90.805) (width 0.25) (layer F.Cu) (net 24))
 (via (at 146.304 82.296) (size 0.6) (layers F.Cu B.Cu) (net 24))
 (via (at 147.828 85.725) (size 0.6) (layers F.Cu B.Cu) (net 24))
 (segment (start 141.985 77.44) (end 141.985 81.152) (width 0.25) (layer F.Cu) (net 12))
 (segment (start 141.985 81.152) (end 144.653 83.82) (width 0.25) (layer F.Cu) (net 12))
 (segment (start 144.653 83.82) (end 151.765 83.82) (width 0.25) (layer F.Cu) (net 12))
 (segment (start 153.67 85.09) (end 147.828 79.248) (width 0.25) (layer B.Cu) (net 17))
 (segment (start 147.828 79.248) (end 134.62 79.248) (width 0.25) (layer B.Cu) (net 17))
 (segment (start 134.62 79.248) (end 133.985 78.613) (width 0.25) (layer F.Cu) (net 17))
 (segment (start 133.985 78.613) (end 133.985 77.44) (width 0.25) (layer F.Cu) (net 17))
 (segment (start 158.115 85.09) (end 153.67 85.09) (width 0.25) (layer F.Cu) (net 17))
 (via (at 153.67 85.09) (size 0.6) (layers F.Cu B.Cu) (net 17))
 (via (at 134.62 79.248) (size 0.6) (layers F.Cu B.Cu) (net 17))
 (segment (start 135.985 77.44) (end 135.985 79.597) (width 0.25) (layer F.Cu) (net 18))
 (segment (start 135.985 79.597) (end 136.525 80.137) (width 0.25) (layer F.Cu) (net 18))
 (segment (start 136.525 80.137) (end 142.875 86.487) (width 0.25) (layer B.Cu) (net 18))
 (segment (start 142.875 86.487) (end 153.543 86.487) (width 0.25) (layer B.Cu) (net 18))
 (segment (start 153.543 86.487) (end 153.67 86.36) (width 0.25) (layer F.Cu) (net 18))
 (segment (start 153.67 86.36) (end 158.115 86.36) (width 0.25) (layer F.Cu) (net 18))
 (via (at 136.525 80.137) (size 0.6) (layers F.Cu B.Cu) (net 18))
 (via (at 153.543 86.487) (size 0.6) (layers F.Cu B.Cu) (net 18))
 (segment (start 132.177 96.2637) (end 132.1766 96.2637) (width 0.25) (layer F.Cu) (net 10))
 (segment (start 132.177 96.2637) (end 132.209 96.2637) (width 0.25) (layer F.Cu) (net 10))
 (segment (start 132.209 96.2637) (end 133.985 94.488) (width 0.25) (layer F.Cu) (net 10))
 (segment (start 133.985 94.488) (end 133.985 91.44) (width 0.25) (layer F.Cu) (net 10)))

